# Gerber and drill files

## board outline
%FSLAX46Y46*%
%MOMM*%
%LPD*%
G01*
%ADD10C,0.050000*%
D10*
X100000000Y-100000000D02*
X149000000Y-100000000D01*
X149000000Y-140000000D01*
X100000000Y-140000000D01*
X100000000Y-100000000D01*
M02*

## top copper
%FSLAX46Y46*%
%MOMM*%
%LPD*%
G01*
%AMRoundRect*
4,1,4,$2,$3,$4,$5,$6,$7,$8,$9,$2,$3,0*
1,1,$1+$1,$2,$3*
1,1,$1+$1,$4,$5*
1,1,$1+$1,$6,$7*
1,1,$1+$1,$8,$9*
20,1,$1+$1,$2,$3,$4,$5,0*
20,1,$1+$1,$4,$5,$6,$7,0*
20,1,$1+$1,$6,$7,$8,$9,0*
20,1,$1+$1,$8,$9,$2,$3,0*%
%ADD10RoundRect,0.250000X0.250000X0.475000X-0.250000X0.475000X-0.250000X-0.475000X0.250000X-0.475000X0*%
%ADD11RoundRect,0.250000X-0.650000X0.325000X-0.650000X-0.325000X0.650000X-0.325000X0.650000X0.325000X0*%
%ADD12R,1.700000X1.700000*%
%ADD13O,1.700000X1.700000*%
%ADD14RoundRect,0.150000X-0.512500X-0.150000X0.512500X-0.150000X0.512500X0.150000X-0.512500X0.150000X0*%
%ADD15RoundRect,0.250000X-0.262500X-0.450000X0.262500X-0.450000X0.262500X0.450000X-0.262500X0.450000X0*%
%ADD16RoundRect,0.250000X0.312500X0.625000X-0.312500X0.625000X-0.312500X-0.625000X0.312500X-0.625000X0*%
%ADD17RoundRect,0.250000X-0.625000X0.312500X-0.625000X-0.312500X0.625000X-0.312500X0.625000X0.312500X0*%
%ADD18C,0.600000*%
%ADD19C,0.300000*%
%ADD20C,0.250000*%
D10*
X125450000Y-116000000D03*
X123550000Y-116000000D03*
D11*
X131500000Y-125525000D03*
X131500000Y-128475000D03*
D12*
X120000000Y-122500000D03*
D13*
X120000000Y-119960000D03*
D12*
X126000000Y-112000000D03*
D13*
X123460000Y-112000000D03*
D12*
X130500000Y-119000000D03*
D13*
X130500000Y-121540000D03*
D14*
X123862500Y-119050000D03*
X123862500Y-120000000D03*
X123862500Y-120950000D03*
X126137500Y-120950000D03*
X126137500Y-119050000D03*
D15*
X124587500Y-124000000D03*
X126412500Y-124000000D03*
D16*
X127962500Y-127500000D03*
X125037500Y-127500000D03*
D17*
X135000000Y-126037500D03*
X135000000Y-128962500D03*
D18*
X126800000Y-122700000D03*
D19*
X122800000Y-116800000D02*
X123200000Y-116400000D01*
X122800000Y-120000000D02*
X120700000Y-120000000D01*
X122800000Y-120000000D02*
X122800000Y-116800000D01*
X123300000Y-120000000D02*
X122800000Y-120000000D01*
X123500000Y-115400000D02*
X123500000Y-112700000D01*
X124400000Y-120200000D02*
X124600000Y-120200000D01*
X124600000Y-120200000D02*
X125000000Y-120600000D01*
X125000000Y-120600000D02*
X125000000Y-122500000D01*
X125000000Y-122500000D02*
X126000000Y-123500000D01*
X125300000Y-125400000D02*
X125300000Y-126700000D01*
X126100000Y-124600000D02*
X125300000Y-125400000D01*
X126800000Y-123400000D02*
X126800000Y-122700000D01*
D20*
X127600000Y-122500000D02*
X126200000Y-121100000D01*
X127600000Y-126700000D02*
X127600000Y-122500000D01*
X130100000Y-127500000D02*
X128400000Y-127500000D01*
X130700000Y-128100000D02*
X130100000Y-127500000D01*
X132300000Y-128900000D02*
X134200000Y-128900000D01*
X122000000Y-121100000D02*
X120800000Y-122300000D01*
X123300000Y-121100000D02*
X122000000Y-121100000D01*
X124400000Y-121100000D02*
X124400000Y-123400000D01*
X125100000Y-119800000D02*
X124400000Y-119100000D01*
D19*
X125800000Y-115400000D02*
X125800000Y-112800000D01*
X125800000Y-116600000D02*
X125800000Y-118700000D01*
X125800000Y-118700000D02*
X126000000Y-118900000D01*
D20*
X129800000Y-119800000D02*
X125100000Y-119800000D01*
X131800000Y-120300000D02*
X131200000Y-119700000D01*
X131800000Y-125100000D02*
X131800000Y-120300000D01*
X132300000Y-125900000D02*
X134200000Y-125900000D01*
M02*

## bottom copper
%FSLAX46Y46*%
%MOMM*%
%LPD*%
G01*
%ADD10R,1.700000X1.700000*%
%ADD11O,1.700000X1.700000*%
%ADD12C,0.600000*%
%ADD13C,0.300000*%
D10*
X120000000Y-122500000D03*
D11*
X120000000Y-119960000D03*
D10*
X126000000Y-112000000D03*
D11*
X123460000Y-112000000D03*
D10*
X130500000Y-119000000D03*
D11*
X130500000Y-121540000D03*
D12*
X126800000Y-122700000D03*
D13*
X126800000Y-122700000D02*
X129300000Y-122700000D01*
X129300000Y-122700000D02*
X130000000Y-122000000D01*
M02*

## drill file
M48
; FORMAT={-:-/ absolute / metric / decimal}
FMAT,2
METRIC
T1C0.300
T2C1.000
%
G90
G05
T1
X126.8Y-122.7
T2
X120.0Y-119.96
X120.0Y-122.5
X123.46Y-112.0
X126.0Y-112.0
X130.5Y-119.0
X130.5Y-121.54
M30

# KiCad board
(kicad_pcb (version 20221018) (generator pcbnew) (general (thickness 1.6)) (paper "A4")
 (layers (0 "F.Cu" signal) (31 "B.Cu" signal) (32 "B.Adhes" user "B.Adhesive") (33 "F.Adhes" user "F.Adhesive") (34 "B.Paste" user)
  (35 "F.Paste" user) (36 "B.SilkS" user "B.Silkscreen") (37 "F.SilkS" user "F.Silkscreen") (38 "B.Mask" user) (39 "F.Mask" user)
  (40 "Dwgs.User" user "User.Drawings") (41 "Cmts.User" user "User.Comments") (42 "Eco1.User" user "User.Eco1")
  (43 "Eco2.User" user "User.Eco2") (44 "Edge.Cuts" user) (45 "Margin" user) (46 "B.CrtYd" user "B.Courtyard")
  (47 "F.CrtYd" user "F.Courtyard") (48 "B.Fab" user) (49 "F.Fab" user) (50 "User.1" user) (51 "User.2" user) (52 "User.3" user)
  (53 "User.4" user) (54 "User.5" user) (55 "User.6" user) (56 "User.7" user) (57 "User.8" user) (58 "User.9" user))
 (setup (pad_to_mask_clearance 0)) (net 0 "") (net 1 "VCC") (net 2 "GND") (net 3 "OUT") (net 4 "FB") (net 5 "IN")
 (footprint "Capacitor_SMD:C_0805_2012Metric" (layer "F.Cu") (at 124.5 116 180)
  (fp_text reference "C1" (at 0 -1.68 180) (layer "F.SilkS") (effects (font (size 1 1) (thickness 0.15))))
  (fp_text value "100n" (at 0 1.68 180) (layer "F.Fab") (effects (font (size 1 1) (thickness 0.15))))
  (pad "1" smd roundrect (at -0.95 0 180) (size 1 1.45) (layers "F.Cu" "F.Paste" "F.Mask") (roundrect_rratio 0.25) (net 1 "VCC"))
  (pad "2" smd roundrect (at 0.95 0 180) (size 1 1.45) (layers "F.Cu" "F.Paste" "F.Mask") (roundrect_rratio 0.25) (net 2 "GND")))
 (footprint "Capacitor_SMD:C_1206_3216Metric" (layer "F.Cu") (at 131.5 127 -90)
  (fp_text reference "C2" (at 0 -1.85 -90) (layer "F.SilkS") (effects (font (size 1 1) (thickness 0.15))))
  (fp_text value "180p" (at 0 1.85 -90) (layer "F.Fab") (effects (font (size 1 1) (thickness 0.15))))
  (pad "1" smd roundrect (at -1.475 0 270) (size 1.15 1.8) (layers "F.Cu" "F.Paste" "F.Mask") (roundrect_rratio 0.217391) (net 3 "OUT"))
  (pad "2" smd roundrect (at 1.475 0 270) (size 1.15 1.8) (layers "F.Cu" "F.Paste" "F.Mask") (roundrect_rratio 0.217391) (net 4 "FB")))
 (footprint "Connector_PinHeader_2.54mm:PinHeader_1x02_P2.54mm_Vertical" (layer "F.Cu") (at 120 122.5 180)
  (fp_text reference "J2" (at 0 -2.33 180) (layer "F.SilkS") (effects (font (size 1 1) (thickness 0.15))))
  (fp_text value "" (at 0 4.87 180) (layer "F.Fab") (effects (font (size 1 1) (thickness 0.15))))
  (pad "1" thru_hole rect (at 0 0 180) (size 1.7 1.7) (drill 1) (layers "*.Cu" "*.Mask") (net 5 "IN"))
  (pad "2" thru_hole oval (at 0 2.54 180) (size 1.7 1.7) (drill 1) (layers "*.Cu" "*.Mask") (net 2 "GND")))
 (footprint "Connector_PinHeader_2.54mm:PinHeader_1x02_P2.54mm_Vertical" (layer "F.Cu") (at 126 112 -90)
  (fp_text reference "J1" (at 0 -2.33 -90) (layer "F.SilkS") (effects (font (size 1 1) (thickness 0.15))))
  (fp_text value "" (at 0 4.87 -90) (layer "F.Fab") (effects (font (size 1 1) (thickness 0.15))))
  (pad "1" thru_hole rect (at 0 0 270) (size 1.7 1.7) (drill 1) (layers "*.Cu" "*.Mask") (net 1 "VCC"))
  (pad "2" thru_hole oval (at 0 2.54 270) (size 1.7 1.7) (drill 1) (layers "*.Cu" "*.Mask") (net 2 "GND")))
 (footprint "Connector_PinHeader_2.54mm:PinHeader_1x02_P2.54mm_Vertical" (layer "F.Cu") (at 130.5 119)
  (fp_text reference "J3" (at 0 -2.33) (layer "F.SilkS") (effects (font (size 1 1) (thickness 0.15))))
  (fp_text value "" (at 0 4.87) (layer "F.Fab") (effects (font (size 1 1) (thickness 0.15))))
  (pad "1" thru_hole rect (at 0 0) (size 1.7 1.7) (drill 1) (layers "*.Cu" "*.Mask") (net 3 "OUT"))
  (pad "2" thru_hole oval (at 0 2.54) (size 1.7 1.7) (drill 1) (layers "*.Cu" "*.Mask") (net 2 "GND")))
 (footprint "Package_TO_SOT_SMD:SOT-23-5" (layer "F.Cu") (at 125 120)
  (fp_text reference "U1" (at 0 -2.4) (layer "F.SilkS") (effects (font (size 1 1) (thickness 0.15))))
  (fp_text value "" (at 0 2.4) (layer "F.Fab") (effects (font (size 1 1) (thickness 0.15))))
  (pad "1" smd roundrect (at -1.1375 -0.95) (size 1.325 0.6) (layers "F.Cu" "F.Paste" "F.Mask") (roundrect_rratio 0.25) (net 3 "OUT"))
  (pad "2" smd roundrect (at -1.1375 0) (size 1.325 0.6) (layers "F.Cu" "F.Paste" "F.Mask") (roundrect_rratio 0.25) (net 2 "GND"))
  (pad "3" smd roundrect (at -1.1375 0.95) (size 1.325 0.6) (layers "F.Cu" "F.Paste" "F.Mask") (roundrect_rratio 0.25) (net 5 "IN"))
  (pad "4" smd roundrect (at 1.1375 0.95) (size 1.325 0.6) (layers "F.Cu" "F.Paste" "F.Mask") (roundrect_rratio 0.25) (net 4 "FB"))
  (pad "5" smd roundrect (at 1.1375 -0.95) (size 1.325 0.6) (layers "F.Cu" "F.Paste" "F.Mask") (roundrect_rratio 0.25) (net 1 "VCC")))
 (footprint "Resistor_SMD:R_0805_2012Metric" (layer "F.Cu") (at 125.5 124)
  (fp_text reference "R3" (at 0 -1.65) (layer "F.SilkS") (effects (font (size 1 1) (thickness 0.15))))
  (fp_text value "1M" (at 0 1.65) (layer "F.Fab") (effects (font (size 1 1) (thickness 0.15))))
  (pad "1" smd roundrect (at -0.9125 0) (size 1.025 1.4) (layers "F.Cu" "F.Paste" "F.Mask") (roundrect_rratio 0.243902) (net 5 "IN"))
  (pad "2" smd roundrect (at 0.9125 0) (size 1.025 1.4) (layers "F.Cu" "F.Paste" "F.Mask") (roundrect_rratio 0.243902) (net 2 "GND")))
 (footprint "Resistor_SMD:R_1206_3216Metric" (layer "F.Cu") (at 126.5 127.5 180)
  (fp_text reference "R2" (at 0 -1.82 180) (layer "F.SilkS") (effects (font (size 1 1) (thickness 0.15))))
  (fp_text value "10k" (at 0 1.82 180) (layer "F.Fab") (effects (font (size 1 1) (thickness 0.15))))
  (pad "1" smd roundrect (at -1.4625 0 180) (size 1.125 1.75) (layers "F.Cu" "F.Paste" "F.Mask") (roundrect_rratio 0.222222) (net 4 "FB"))
  (pad "2" smd roundrect (at 1.4625 0 180) (size 1.125 1.75) (layers "F.Cu" "F.Paste" "F.Mask") (roundrect_rratio 0.222222) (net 2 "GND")))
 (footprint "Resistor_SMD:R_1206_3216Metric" (layer "F.Cu") (at 135 127.5 -90)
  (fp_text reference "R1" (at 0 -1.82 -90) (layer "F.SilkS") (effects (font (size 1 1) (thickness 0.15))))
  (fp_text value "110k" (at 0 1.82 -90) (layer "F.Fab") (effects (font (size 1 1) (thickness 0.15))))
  (pad "1" smd roundrect (at -1.4625 0 270) (size 1.125 1.75) (layers "F.Cu" "F.Paste" "F.Mask") (roundrect_rratio 0.222222) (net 3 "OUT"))
  (pad "2" smd roundrect (at 1.4625 0 270) (size 1.125 1.75) (layers "F.Cu" "F.Paste" "F.Mask") (roundrect_rratio 0.222222) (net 4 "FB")))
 (gr_rect (start 100 100) (end 149 140) (stroke (width 0.05) (type default)) (fill none) (layer "Edge.Cuts"))
 (segment (start 122.8 116.8) (end 123.2 116.4) (width 0.3) (layer "F.Cu") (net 2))
 (segment (start 122.8 120) (end 120.7 120) (width 0.3) (layer "F.Cu") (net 2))
 (segment (start 122.8 120) (end 122.8 116.8) (width 0.3) (layer "F.Cu") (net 2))
 (segment (start 123.3 120) (end 122.8 120) (width 0.3) (layer "F.Cu") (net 2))
 (segment (start 123.5 115.4) (end 123.5 112.7) (width 0.3) (layer "F.Cu") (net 2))
 (segment (start 124.4 120.2) (end 124.6 120.2) (width 0.3) (layer "F.Cu") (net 2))
 (segment (start 124.6 120.2) (end 125 120.6) (width 0.3) (layer "F.Cu") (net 2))
 (segment (start 125 120.6) (end 125 122.5) (width 0.3) (layer "F.Cu") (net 2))
 (segment (start 125 122.5) (end 126 123.5) (width 0.3) (layer "F.Cu") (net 2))
 (segment (start 125.3 125.4) (end 125.3 126.7) (width 0.3) (layer "F.Cu") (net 2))
 (segment (start 126.1 124.6) (end 125.3 125.4) (width 0.3) (layer "F.Cu") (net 2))
 (segment (start 126.8 123.4) (end 126.8 122.7) (width 0.3) (layer "F.Cu") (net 2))
 (segment (start 127.6 122.5) (end 126.2 121.1) (width 0.25) (layer "F.Cu") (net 4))
 (segment (start 127.6 126.7) (end 127.6 122.5) (width 0.25) (layer "F.Cu") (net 4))
 (segment (start 130.1 127.5) (end 128.4 127.5) (width 0.25) (layer "F.Cu") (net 4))
 (segment (start 130.7 128.1) (end 130.1 127.5) (width 0.25) (layer "F.Cu") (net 4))
 (segment (start 132.3 128.9) (end 134.2 128.9) (width 0.25) (layer "F.Cu") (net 4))
 (via (at 126.8 122.7) (size 0.6) (drill 0.3) (layers "F.Cu" "B.Cu") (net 2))
 (segment (start 122 121.1) (end 120.8 122.3) (width 0.25) (layer "F.Cu") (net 5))
 (segment (start 123.3 121.1) (end 122 121.1) (width 0.25) (layer "F.Cu") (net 5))
 (segment (start 124.4 121.1) (end 124.4 123.4) (width 0.25) (layer "F.Cu") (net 5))
 (segment (start 125.1 119.8) (end 124.4 119.1) (width 0.25) (layer "F.Cu") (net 3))
 (segment (start 125.8 115.4) (end 125.8 112.8) (width 0.3) (layer "F.Cu") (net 1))
 (segment (start 125.8 116.6) (end 125.8 118.7) (width 0.3) (layer "F.Cu") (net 1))
 (segment (start 125.8 118.7) (end 126 118.9) (width 0.3) (layer "F.Cu") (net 1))
 (segment (start 126.8 122.7) (end 129.3 122.7) (width 0.3) (layer "B.Cu") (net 2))
 (segment (start 129.3 122.7) (end 130 122) (width 0.3) (layer "B.Cu") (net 2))
 (segment (start 129.8 119.8) (end 125.1 119.8) (width 0.25) (layer "F.Cu") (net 3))
 (segment (start 131.8 120.3) (end 131.2 119.7) (width 0.25) (layer "F.Cu") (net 3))
 (segment (start 131.8 125.1) (end 131.8 120.3) (width 0.25) (layer "F.Cu") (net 3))
 (segment (start 132.3 125.9) (end 134.2 125.9) (width 0.25) (layer "F.Cu") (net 3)))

